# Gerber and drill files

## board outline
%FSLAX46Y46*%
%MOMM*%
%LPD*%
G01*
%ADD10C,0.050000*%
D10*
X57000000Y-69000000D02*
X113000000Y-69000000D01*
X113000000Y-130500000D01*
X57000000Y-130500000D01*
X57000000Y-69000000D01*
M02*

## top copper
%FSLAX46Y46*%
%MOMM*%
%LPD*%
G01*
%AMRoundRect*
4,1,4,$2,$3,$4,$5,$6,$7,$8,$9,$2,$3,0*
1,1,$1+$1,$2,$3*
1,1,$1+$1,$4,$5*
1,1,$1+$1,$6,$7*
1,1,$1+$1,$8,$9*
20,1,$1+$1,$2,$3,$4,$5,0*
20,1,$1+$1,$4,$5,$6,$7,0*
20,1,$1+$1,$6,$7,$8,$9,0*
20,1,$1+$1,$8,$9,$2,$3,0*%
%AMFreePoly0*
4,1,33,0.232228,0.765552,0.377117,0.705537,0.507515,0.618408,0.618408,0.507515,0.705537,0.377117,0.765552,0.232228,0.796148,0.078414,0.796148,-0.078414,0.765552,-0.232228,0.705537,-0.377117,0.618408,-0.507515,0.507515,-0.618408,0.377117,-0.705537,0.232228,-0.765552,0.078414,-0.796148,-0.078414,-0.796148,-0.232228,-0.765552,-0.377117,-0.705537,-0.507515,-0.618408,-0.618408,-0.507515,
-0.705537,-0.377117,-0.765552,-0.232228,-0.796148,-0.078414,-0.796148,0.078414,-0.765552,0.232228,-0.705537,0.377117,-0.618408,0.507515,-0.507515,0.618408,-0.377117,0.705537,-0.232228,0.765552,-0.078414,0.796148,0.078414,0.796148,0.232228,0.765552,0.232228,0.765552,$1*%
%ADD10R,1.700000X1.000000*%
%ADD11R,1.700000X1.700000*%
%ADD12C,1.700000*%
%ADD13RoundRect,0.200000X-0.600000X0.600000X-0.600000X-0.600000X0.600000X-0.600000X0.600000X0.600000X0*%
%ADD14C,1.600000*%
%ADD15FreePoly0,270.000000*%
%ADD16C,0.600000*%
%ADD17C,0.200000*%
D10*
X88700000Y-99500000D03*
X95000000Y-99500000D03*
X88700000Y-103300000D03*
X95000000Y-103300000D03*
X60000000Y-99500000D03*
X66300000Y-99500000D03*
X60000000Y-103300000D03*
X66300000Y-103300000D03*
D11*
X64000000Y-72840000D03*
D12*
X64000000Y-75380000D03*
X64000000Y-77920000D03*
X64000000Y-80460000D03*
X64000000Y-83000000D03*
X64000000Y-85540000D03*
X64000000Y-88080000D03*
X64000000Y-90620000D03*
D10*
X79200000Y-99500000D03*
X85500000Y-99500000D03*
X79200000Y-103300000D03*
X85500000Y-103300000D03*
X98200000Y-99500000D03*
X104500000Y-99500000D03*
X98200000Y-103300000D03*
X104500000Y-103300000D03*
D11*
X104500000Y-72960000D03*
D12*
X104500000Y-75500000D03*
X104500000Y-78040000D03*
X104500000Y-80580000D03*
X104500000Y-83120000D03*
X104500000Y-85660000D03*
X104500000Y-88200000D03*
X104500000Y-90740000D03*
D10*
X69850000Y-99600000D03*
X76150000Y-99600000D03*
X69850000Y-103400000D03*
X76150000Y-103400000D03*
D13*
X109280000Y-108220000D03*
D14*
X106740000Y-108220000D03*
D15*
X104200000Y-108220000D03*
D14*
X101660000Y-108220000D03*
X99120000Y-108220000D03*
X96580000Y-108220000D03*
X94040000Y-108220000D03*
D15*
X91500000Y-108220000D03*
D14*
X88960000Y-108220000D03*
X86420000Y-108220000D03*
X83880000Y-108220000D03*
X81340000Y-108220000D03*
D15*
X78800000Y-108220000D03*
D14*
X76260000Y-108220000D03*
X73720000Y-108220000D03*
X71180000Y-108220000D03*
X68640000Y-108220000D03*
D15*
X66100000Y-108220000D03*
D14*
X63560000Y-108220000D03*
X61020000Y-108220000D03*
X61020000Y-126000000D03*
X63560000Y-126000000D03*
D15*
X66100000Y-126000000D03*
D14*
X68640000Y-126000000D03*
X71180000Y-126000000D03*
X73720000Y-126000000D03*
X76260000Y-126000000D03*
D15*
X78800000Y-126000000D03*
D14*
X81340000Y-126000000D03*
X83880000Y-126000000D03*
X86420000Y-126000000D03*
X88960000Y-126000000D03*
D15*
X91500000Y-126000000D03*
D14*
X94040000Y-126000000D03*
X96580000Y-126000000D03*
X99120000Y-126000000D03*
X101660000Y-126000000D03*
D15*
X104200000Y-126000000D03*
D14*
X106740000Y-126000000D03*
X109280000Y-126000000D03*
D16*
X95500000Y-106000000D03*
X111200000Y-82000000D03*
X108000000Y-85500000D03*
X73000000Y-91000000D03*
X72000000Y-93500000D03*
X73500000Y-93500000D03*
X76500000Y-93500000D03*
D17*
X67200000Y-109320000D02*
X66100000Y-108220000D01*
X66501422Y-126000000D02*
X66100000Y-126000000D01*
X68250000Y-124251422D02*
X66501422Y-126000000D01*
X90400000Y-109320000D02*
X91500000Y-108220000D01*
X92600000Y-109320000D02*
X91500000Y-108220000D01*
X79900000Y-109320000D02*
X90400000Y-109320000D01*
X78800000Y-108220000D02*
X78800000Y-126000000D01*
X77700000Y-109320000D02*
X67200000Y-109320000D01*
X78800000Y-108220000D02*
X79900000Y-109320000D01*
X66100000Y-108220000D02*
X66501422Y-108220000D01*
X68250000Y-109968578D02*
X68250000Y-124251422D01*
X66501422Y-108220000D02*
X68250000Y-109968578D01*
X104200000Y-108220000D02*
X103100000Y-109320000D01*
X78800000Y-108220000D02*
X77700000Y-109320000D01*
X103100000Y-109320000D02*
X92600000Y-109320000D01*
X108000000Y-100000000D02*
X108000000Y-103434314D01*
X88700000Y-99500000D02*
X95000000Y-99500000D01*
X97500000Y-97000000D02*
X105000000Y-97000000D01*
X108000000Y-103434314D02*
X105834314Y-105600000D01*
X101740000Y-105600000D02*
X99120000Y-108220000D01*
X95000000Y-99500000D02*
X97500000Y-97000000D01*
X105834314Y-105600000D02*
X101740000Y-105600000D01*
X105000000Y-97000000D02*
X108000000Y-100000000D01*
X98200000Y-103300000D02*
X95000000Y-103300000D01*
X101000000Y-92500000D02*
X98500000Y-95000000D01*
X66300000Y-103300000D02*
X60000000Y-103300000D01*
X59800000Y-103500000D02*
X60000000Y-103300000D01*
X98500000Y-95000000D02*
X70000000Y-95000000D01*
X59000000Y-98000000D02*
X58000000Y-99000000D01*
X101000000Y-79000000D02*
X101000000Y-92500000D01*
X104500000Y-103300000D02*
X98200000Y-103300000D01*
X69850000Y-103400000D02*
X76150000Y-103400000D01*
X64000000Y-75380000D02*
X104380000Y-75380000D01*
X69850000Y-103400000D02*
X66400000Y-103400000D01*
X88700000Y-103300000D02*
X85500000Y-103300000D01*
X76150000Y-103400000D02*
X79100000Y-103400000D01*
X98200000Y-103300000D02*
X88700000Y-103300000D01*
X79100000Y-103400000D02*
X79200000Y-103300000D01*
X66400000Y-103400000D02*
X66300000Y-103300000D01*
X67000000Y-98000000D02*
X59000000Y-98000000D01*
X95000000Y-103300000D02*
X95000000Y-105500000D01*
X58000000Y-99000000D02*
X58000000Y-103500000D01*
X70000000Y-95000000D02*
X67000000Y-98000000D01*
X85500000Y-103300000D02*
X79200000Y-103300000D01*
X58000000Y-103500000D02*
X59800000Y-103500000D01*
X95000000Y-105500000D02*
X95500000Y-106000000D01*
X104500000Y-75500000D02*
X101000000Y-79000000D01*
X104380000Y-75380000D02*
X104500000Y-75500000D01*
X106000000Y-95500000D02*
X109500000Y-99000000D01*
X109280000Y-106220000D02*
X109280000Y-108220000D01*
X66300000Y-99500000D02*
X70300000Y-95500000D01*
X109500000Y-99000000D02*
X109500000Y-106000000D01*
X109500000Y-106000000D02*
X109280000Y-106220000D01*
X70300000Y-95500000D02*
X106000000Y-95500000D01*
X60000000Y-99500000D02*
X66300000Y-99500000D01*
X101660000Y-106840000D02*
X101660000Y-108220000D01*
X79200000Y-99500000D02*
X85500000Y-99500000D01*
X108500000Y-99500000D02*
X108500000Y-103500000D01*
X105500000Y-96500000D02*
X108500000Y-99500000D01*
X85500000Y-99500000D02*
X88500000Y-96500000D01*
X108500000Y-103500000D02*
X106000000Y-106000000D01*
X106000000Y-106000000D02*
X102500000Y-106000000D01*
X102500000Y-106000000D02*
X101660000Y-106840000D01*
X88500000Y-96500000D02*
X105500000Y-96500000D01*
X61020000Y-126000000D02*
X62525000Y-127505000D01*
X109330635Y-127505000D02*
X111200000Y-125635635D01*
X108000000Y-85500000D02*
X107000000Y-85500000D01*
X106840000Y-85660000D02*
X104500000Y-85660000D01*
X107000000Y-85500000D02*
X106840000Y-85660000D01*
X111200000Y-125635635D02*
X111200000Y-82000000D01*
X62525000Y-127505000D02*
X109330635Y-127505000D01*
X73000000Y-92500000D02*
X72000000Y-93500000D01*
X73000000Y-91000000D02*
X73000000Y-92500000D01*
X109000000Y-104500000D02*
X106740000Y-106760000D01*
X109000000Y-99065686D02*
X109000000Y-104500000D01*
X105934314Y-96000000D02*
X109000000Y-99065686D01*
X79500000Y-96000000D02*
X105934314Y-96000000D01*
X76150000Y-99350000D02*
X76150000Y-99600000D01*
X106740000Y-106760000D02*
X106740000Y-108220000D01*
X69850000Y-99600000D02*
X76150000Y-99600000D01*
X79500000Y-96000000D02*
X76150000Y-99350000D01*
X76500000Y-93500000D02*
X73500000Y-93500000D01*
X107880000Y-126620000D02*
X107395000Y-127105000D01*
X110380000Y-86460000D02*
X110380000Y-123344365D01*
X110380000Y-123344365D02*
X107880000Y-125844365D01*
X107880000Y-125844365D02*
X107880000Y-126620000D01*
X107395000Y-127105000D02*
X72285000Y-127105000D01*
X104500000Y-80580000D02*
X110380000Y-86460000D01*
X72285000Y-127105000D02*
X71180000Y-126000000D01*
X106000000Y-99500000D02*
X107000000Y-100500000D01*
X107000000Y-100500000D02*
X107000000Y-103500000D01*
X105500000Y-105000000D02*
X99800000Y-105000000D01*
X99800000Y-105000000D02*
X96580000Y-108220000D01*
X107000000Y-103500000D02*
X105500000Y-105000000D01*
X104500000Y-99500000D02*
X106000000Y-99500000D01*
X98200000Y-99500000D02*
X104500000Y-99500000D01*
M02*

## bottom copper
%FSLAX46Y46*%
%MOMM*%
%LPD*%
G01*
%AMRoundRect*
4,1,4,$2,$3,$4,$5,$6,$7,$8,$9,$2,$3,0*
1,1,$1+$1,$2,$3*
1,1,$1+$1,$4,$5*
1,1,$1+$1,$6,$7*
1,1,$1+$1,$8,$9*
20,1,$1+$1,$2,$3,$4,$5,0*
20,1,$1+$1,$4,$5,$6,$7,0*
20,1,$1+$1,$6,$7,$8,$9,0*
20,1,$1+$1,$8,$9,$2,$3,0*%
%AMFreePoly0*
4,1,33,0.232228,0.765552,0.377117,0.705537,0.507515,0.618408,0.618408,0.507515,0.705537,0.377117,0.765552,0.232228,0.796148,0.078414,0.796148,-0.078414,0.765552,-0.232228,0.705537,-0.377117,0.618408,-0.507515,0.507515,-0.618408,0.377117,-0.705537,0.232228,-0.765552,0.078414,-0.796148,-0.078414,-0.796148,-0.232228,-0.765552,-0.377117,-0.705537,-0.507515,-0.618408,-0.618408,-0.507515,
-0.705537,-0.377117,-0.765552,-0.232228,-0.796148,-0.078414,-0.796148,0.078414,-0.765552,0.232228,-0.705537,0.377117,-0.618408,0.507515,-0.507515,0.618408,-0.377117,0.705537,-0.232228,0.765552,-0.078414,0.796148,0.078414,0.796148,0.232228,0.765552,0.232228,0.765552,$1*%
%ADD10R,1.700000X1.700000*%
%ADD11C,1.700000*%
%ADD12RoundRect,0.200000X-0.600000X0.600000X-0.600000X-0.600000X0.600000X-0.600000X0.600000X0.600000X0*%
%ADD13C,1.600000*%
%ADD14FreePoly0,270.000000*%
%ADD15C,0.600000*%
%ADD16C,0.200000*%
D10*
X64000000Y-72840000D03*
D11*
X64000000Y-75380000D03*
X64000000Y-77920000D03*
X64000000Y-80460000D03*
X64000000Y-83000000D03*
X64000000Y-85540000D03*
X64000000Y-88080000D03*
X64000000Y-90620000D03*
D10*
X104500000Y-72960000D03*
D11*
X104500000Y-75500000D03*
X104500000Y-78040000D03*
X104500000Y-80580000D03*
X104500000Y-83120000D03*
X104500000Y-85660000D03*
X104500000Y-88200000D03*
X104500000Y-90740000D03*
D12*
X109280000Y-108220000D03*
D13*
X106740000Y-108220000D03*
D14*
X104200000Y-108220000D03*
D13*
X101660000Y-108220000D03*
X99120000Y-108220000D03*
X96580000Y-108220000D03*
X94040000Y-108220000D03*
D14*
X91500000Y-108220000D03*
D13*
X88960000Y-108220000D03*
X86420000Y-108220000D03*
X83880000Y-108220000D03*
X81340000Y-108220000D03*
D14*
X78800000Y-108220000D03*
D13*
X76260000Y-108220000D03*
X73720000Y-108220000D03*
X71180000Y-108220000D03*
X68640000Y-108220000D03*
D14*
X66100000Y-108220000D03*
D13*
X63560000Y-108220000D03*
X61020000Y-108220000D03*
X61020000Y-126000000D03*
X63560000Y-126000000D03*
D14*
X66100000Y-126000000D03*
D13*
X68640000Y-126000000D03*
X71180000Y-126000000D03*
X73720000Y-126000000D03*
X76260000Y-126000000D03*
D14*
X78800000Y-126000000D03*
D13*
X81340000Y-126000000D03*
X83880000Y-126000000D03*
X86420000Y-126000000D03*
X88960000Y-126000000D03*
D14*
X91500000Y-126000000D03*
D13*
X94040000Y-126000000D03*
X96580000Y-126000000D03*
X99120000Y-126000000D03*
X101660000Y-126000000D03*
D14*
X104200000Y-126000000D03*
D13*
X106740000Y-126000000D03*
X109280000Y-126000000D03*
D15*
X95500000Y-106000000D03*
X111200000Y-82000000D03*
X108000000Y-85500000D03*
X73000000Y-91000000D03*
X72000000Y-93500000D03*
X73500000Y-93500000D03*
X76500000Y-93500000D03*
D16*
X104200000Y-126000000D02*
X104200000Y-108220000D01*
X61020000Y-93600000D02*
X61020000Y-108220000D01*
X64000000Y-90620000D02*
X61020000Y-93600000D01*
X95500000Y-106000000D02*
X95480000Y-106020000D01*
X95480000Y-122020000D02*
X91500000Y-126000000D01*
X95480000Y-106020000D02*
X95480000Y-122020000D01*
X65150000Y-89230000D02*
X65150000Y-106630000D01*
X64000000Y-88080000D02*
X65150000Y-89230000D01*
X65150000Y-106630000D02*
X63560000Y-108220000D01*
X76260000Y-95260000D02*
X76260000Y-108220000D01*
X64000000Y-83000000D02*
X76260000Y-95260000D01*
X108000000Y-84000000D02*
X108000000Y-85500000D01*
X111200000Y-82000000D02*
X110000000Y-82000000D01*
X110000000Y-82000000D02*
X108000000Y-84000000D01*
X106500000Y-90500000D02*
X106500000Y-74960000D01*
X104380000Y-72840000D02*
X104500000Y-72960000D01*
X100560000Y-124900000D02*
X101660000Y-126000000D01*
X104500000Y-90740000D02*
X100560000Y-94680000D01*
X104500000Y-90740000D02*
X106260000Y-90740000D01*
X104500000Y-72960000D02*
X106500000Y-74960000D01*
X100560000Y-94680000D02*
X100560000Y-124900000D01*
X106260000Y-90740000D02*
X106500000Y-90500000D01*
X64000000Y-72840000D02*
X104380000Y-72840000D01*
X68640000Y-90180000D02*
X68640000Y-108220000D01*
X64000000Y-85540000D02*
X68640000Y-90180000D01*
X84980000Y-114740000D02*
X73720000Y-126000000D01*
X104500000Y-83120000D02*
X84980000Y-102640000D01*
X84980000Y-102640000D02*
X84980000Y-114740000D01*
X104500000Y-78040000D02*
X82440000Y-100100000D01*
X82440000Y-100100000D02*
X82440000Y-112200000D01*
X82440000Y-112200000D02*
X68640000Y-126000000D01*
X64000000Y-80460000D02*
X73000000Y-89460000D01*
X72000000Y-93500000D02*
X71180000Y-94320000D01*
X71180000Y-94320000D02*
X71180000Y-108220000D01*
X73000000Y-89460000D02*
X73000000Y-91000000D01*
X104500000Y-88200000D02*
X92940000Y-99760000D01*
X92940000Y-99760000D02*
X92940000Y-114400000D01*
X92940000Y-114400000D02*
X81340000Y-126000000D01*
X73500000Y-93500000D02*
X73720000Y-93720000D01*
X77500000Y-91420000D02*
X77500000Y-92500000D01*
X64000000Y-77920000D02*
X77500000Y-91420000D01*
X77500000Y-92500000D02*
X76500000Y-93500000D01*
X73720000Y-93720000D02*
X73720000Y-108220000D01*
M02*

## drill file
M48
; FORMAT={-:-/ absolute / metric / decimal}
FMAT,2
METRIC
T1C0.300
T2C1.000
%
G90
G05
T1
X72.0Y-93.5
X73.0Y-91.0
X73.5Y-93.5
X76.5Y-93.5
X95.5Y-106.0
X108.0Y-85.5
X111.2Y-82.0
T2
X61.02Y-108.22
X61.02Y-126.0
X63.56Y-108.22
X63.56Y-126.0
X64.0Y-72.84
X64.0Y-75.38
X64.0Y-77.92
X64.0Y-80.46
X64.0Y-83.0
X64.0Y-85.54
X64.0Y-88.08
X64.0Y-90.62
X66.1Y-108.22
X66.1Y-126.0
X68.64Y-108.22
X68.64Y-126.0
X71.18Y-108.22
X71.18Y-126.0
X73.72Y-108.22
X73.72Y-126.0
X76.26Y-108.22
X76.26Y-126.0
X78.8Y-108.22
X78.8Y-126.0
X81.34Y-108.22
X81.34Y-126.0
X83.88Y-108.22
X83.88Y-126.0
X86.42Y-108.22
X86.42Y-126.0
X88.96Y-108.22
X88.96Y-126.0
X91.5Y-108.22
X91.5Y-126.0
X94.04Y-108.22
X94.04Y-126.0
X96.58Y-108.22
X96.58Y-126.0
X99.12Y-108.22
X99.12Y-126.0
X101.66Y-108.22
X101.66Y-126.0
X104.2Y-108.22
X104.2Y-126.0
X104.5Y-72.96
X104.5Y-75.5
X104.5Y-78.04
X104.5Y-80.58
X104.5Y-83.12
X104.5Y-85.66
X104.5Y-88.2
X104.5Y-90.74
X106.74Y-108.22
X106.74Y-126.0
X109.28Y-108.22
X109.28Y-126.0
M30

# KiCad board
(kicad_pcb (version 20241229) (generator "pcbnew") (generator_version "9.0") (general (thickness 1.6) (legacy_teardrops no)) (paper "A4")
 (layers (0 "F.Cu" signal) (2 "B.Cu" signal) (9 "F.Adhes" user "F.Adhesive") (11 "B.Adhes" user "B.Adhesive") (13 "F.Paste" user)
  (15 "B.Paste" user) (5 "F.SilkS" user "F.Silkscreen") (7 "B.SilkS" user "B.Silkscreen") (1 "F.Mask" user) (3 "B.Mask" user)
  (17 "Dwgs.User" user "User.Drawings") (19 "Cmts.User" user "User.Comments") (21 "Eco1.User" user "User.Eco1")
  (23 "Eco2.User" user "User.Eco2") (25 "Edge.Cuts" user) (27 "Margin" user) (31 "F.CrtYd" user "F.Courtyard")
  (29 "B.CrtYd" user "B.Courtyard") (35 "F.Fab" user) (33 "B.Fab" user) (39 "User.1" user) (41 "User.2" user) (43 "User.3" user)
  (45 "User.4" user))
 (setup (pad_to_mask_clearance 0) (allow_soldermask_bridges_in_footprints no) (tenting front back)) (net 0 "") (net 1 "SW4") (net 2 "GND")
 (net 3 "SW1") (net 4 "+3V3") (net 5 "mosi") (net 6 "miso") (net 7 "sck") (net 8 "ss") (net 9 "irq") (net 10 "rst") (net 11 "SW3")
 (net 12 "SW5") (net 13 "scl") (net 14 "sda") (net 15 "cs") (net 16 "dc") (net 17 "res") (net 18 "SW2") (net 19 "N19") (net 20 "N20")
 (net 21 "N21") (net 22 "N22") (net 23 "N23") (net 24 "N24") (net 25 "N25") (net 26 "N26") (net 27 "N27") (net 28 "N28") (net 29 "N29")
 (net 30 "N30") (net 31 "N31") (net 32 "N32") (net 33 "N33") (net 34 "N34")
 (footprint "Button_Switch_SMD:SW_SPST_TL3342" (layer "F.Cu") (at 91.85 101.4)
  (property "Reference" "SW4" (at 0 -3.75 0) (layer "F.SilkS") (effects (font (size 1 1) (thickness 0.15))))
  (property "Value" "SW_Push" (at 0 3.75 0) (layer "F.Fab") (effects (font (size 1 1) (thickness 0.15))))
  (pad "1" smd rect (at -3.15 -1.9) (size 1.7 1) (layers "F.Cu" "F.Mask" "F.Paste") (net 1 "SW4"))
  (pad "1" smd rect (at 3.15 -1.9) (size 1.7 1) (layers "F.Cu" "F.Mask" "F.Paste") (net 1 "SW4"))
  (pad "2" smd rect (at -3.15 1.9) (size 1.7 1) (layers "F.Cu" "F.Mask" "F.Paste") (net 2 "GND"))
  (pad "2" smd rect (at 3.15 1.9) (size 1.7 1) (layers "F.Cu" "F.Mask" "F.Paste") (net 2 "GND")))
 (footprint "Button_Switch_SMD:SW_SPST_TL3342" (layer "F.Cu") (at 63.15 101.4)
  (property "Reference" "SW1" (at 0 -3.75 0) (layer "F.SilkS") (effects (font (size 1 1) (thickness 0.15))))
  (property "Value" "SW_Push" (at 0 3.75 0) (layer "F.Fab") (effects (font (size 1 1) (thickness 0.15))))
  (pad "1" smd rect (at -3.15 -1.9) (size 1.7 1) (layers "F.Cu" "F.Mask" "F.Paste") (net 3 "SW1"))
  (pad "1" smd rect (at 3.15 -1.9) (size 1.7 1) (layers "F.Cu" "F.Mask" "F.Paste") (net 3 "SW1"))
  (pad "2" smd rect (at -3.15 1.9) (size 1.7 1) (layers "F.Cu" "F.Mask" "F.Paste") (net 2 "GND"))
  (pad "2" smd rect (at 3.15 1.9) (size 1.7 1) (layers "F.Cu" "F.Mask" "F.Paste") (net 2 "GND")))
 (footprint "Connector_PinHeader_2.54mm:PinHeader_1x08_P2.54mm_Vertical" (layer "F.Cu") (at 64 72.84)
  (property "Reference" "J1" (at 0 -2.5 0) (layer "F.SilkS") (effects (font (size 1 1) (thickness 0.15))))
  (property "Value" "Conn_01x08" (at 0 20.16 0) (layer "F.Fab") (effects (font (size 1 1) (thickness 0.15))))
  (pad "1" thru_hole rect (at 0 0) (size 1.7 1.7) (drill 1) (layers "*.Cu" "*.Mask") (remove_unused_layers no) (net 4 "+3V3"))
  (pad "2" thru_hole circle (at 0 2.54) (size 1.7 1.7) (drill 1) (layers "*.Cu" "*.Mask") (remove_unused_layers no) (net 2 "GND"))
  (pad "3" thru_hole circle (at 0 5.08) (size 1.7 1.7) (drill 1) (layers "*.Cu" "*.Mask") (remove_unused_layers no) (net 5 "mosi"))
  (pad "4" thru_hole circle (at 0 7.62) (size 1.7 1.7) (drill 1) (layers "*.Cu" "*.Mask") (remove_unused_layers no) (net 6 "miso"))
  (pad "5" thru_hole circle (at 0 10.16) (size 1.7 1.7) (drill 1) (layers "*.Cu" "*.Mask") (remove_unused_layers no) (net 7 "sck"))
  (pad "6" thru_hole circle (at 0 12.7) (size 1.7 1.7) (drill 1) (layers "*.Cu" "*.Mask") (remove_unused_layers no) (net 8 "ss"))
  (pad "7" thru_hole circle (at 0 15.24) (size 1.7 1.7) (drill 1) (layers "*.Cu" "*.Mask") (remove_unused_layers no) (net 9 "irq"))
  (pad "8" thru_hole circle (at 0 17.78) (size 1.7 1.7) (drill 1) (layers "*.Cu" "*.Mask") (remove_unused_layers no) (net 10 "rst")))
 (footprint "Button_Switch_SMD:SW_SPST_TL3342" (layer "F.Cu") (at 82.35 101.4)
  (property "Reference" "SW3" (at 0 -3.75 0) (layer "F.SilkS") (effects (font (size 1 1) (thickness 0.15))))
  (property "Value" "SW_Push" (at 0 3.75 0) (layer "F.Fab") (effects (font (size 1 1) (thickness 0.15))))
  (pad "1" smd rect (at -3.15 -1.9) (size 1.7 1) (layers "F.Cu" "F.Mask" "F.Paste") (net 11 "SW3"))
  (pad "1" smd rect (at 3.15 -1.9) (size 1.7 1) (layers "F.Cu" "F.Mask" "F.Paste") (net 11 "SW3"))
  (pad "2" smd rect (at -3.15 1.9) (size 1.7 1) (layers "F.Cu" "F.Mask" "F.Paste") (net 2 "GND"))
  (pad "2" smd rect (at 3.15 1.9) (size 1.7 1) (layers "F.Cu" "F.Mask" "F.Paste") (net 2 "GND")))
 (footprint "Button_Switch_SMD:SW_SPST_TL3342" (layer "F.Cu") (at 101.35 101.4)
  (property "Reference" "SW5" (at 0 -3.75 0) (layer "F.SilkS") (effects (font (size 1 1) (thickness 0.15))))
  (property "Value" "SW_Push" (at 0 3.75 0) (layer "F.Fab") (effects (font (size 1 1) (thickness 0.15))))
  (pad "1" smd rect (at -3.15 -1.9) (size 1.7 1) (layers "F.Cu" "F.Mask" "F.Paste") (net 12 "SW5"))
  (pad "1" smd rect (at 3.15 -1.9) (size 1.7 1) (layers "F.Cu" "F.Mask" "F.Paste") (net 12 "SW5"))
  (pad "2" smd rect (at -3.15 1.9) (size 1.7 1) (layers "F.Cu" "F.Mask" "F.Paste") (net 2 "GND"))
  (pad "2" smd rect (at 3.15 1.9) (size 1.7 1) (layers "F.Cu" "F.Mask" "F.Paste") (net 2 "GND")))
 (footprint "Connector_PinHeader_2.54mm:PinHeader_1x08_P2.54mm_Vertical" (layer "F.Cu") (at 104.5 72.96)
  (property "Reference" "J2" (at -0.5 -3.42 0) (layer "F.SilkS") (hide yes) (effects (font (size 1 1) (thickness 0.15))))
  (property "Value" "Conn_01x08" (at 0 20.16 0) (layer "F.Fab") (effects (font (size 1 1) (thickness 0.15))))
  (pad "1" thru_hole rect (at 0 0) (size 1.7 1.7) (drill 1) (layers "*.Cu" "*.Mask") (remove_unused_layers no) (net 4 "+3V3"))
  (pad "2" thru_hole circle (at 0 2.54) (size 1.7 1.7) (drill 1) (layers "*.Cu" "*.Mask") (remove_unused_layers no) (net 2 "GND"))
  (pad "3" thru_hole circle (at 0 5.08) (size 1.7 1.7) (drill 1) (layers "*.Cu" "*.Mask") (remove_unused_layers no) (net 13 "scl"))
  (pad "4" thru_hole circle (at 0 7.62) (size 1.7 1.7) (drill 1) (layers "*.Cu" "*.Mask") (remove_unused_layers no) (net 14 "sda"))
  (pad "5" thru_hole circle (at 0 10.16) (size 1.7 1.7) (drill 1) (layers "*.Cu" "*.Mask") (remove_unused_layers no) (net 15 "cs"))
  (pad "6" thru_hole circle (at 0 12.7) (size 1.7 1.7) (drill 1) (layers "*.Cu" "*.Mask") (remove_unused_layers no) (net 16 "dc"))
  (pad "7" thru_hole circle (at 0 15.24) (size 1.7 1.7) (drill 1) (layers "*.Cu" "*.Mask") (remove_unused_layers no) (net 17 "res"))
  (pad "8" thru_hole circle (at 0 17.78) (size 1.7 1.7) (drill 1) (layers "*.Cu" "*.Mask") (remove_unused_layers no) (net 4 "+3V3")))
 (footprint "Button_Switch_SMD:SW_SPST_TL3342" (layer "F.Cu") (at 73 101.5)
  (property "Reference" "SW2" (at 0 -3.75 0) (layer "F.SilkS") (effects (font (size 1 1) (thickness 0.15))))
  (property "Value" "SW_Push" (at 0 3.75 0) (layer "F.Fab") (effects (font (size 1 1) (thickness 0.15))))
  (pad "1" smd rect (at -3.15 -1.9) (size 1.7 1) (layers "F.Cu" "F.Mask" "F.Paste") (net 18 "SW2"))
  (pad "1" smd rect (at 3.15 -1.9) (size 1.7 1) (layers "F.Cu" "F.Mask" "F.Paste") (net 18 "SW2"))
  (pad "2" smd rect (at -3.15 1.9) (size 1.7 1) (layers "F.Cu" "F.Mask" "F.Paste") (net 2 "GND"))
  (pad "2" smd rect (at 3.15 1.9) (size 1.7 1) (layers "F.Cu" "F.Mask" "F.Paste") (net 2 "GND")))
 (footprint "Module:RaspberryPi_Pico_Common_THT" (layer "F.Cu") (at 109.28 108.22 -90)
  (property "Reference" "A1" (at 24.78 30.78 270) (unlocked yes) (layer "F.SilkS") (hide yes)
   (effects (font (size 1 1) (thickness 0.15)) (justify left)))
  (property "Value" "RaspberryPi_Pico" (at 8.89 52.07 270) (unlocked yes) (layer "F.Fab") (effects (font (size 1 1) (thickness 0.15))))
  (pad "1" thru_hole roundrect (at 0 0 270) (size 1.6 1.6) (drill 1) (layers "*.Cu" "*.Mask") (remove_unused_layers no)
   (roundrect_rratio 0.125) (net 3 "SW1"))
  (pad "2" thru_hole circle (at 0 2.54 270) (size 1.6 1.6) (drill 1) (layers "*.Cu" "*.Mask") (remove_unused_layers no) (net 18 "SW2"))
  (pad "3" thru_hole custom (at 0 5.08 270) (size 1.6 1.6) (drill 1) (layers "*.Cu" "*.Mask") (remove_unused_layers no) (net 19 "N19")
   (options (clearance outline) (anchor circle)) (primitives))
  (pad "4" thru_hole circle (at 0 7.62 270) (size 1.6 1.6) (drill 1) (layers "*.Cu" "*.Mask") (remove_unused_layers no) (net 11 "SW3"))
  (pad "5" thru_hole circle (at 0 10.16 270) (size 1.6 1.6) (drill 1) (layers "*.Cu" "*.Mask") (remove_unused_layers no) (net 1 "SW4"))
  (pad "6" thru_hole circle (at 0 12.7 270) (size 1.6 1.6) (drill 1) (layers "*.Cu" "*.Mask") (remove_unused_layers no) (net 12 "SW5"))
  (pad "7" thru_hole circle (at 0 15.24 270) (size 1.6 1.6) (drill 1) (layers "*.Cu" "*.Mask") (remove_unused_layers no) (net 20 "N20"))
  (pad "8" thru_hole custom (at 0 17.78 270) (size 1.6 1.6) (drill 1) (layers "*.Cu" "*.Mask") (remove_unused_layers no) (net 19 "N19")
   (options (clearance outline) (anchor circle)) (primitives))
  (pad "9" thru_hole circle (at 0 20.32 270) (size 1.6 1.6) (drill 1) (layers "*.Cu" "*.Mask") (remove_unused_layers no) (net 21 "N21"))
  (pad "10" thru_hole circle (at 0 22.86 270) (size 1.6 1.6) (drill 1) (layers "*.Cu" "*.Mask") (remove_unused_layers no) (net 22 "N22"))
  (pad "11" thru_hole circle (at 0 25.4 270) (size 1.6 1.6) (drill 1) (layers "*.Cu" "*.Mask") (remove_unused_layers no) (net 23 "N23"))
  (pad "12" thru_hole circle (at 0 27.94 270) (size 1.6 1.6) (drill 1) (layers "*.Cu" "*.Mask") (remove_unused_layers no) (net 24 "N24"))
  (pad "13" thru_hole custom (at 0 30.48 270) (size 1.6 1.6) (drill 1) (layers "*.Cu" "*.Mask") (remove_unused_layers no) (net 19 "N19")
   (options (clearance outline) (anchor circle)) (primitives))
  (pad "14" thru_hole circle (at 0 33.02 270) (size 1.6 1.6) (drill 1) (layers "*.Cu" "*.Mask") (remove_unused_layers no) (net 7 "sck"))
  (pad "15" thru_hole circle (at 0 35.56 270) (size 1.6 1.6) (drill 1) (layers "*.Cu" "*.Mask") (remove_unused_layers no) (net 5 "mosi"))
  (pad "16" thru_hole circle (at 0 38.1 270) (size 1.6 1.6) (drill 1) (layers "*.Cu" "*.Mask") (remove_unused_layers no) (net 6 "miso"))
  (pad "17" thru_hole circle (at 0 40.64 270) (size 1.6 1.6) (drill 1) (layers "*.Cu" "*.Mask") (remove_unused_layers no) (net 8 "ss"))
  (pad "18" thru_hole custom (at 0 43.18 270) (size 1.6 1.6) (drill 1) (layers "*.Cu" "*.Mask") (remove_unused_layers no) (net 19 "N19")
   (options (clearance outline) (anchor circle)) (primitives))
  (pad "19" thru_hole circle (at 0 45.72 270) (size 1.6 1.6) (drill 1) (layers "*.Cu" "*.Mask") (remove_unused_layers no) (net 9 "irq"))
  (pad "20" thru_hole circle (at 0 48.26 270) (size 1.6 1.6) (drill 1) (layers "*.Cu" "*.Mask") (remove_unused_layers no) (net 10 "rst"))
  (pad "21" thru_hole circle (at 17.78 48.26 270) (size 1.6 1.6) (drill 1) (layers "*.Cu" "*.Mask") (remove_unused_layers no) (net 16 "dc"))
  (pad "22" thru_hole circle (at 17.78 45.72 270) (size 1.6 1.6) (drill 1) (layers "*.Cu" "*.Mask") (remove_unused_layers no) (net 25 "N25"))
  (pad "23" thru_hole custom (at 17.78 43.18 270) (size 1.6 1.6) (drill 1) (layers "*.Cu" "*.Mask") (remove_unused_layers no) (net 19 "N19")
   (options (clearance outline) (anchor circle)) (primitives))
  (pad "24" thru_hole circle (at 17.78 40.64 270) (size 1.6 1.6) (drill 1) (layers "*.Cu" "*.Mask") (remove_unused_layers no) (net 13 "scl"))
  (pad "25" thru_hole circle (at 17.78 38.1 270) (size 1.6 1.6) (drill 1) (layers "*.Cu" "*.Mask") (remove_unused_layers no) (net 14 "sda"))
  (pad "26" thru_hole circle (at 17.78 35.56 270) (size 1.6 1.6) (drill 1) (layers "*.Cu" "*.Mask") (remove_unused_layers no) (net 15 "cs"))
  (pad "27" thru_hole circle (at 17.78 33.02 270) (size 1.6 1.6) (drill 1) (layers "*.Cu" "*.Mask") (remove_unused_layers no) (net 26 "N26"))
  (pad "28" thru_hole custom (at 17.78 30.48 270) (size 1.6 1.6) (drill 1) (layers "*.Cu" "*.Mask") (remove_unused_layers no) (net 19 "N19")
   (options (clearance outline) (anchor circle)) (primitives))
  (pad "29" thru_hole circle (at 17.78 27.94 270) (size 1.6 1.6) (drill 1) (layers "*.Cu" "*.Mask") (remove_unused_layers no) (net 17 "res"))
  (pad "30" thru_hole circle (at 17.78 25.4 270) (size 1.6 1.6) (drill 1) (layers "*.Cu" "*.Mask") (remove_unused_layers no) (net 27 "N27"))
  (pad "31" thru_hole circle (at 17.78 22.86 270) (size 1.6 1.6) (drill 1) (layers "*.Cu" "*.Mask") (remove_unused_layers no) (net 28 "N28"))
  (pad "32" thru_hole circle (at 17.78 20.32 270) (size 1.6 1.6) (drill 1) (layers "*.Cu" "*.Mask") (remove_unused_layers no) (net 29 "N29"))
  (pad "33" thru_hole custom (at 17.78 17.78 270) (size 1.6 1.6) (drill 1) (layers "*.Cu" "*.Mask") (remove_unused_layers no) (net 2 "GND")
   (options (clearance outline) (anchor circle)) (primitives))
  (pad "34" thru_hole circle (at 17.78 15.24 270) (size 1.6 1.6) (drill 1) (layers "*.Cu" "*.Mask") (remove_unused_layers no) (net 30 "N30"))
  (pad "35" thru_hole circle (at 17.78 12.7 270) (size 1.6 1.6) (drill 1) (layers "*.Cu" "*.Mask") (remove_unused_layers no) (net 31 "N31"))
  (pad "36" thru_hole circle (at 17.78 10.16 270) (size 1.6 1.6) (drill 1) (layers "*.Cu" "*.Mask") (remove_unused_layers no) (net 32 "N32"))
  (pad "37" thru_hole circle (at 17.78 7.62 270) (size 1.6 1.6) (drill 1) (layers "*.Cu" "*.Mask") (remove_unused_layers no) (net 4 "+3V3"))
  (pad "38" thru_hole custom (at 17.78 5.08 270) (size 1.6 1.6) (drill 1) (layers "*.Cu" "*.Mask") (remove_unused_layers no) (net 19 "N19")
   (options (clearance outline) (anchor circle)) (primitives))
  (pad "39" thru_hole circle (at 17.78 2.54 270) (size 1.6 1.6) (drill 1) (layers "*.Cu" "*.Mask") (remove_unused_layers no) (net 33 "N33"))
  (pad "40" thru_hole circle (at 17.78 0 270) (size 1.6 1.6) (drill 1) (layers "*.Cu" "*.Mask") (remove_unused_layers no) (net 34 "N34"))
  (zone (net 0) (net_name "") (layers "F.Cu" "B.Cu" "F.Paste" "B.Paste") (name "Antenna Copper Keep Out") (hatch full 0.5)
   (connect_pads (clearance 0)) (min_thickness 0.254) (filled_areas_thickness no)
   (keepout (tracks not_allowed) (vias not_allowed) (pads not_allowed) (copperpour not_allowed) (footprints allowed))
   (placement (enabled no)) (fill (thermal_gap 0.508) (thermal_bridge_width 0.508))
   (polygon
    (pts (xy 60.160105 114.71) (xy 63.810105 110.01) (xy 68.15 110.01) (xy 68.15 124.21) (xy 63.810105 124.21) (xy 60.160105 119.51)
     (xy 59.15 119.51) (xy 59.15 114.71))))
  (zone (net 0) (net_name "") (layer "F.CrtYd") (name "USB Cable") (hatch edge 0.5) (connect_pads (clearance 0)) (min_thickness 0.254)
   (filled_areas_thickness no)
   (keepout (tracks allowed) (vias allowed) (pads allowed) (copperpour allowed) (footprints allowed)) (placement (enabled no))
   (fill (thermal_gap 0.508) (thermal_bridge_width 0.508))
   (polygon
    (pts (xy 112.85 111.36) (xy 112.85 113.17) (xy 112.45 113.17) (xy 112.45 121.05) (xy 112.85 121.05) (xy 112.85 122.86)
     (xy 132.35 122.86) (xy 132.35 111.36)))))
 (gr_rect (start 57 69) (end 113 130.5) (stroke (width 0.05) (type default)) (fill no) (layer "Edge.Cuts"))
 (segment (start 67.2 109.32) (end 66.1 108.22) (width 0.2) (layer "F.Cu") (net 19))
 (segment (start 66.501422 126) (end 66.1 126) (width 0.2) (layer "F.Cu") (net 19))
 (segment (start 68.25 124.251422) (end 66.501422 126) (width 0.2) (layer "F.Cu") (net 19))
 (segment (start 90.4 109.32) (end 91.5 108.22) (width 0.2) (layer "F.Cu") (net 19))
 (segment (start 92.6 109.32) (end 91.5 108.22) (width 0.2) (layer "F.Cu") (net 19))
 (segment (start 79.9 109.32) (end 90.4 109.32) (width 0.2) (layer "F.Cu") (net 19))
 (segment (start 78.8 108.22) (end 78.8 126) (width 0.2) (layer "F.Cu") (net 19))
 (segment (start 77.7 109.32) (end 67.2 109.32) (width 0.2) (layer "F.Cu") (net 19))
 (segment (start 78.8 108.22) (end 79.9 109.32) (width 0.2) (layer "F.Cu") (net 19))
 (segment (start 66.1 108.22) (end 66.501422 108.22) (width 0.2) (layer "F.Cu") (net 19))
 (segment (start 68.25 109.968578) (end 68.25 124.251422) (width 0.2) (layer "F.Cu") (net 19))
 (segment (start 66.501422 108.22) (end 68.25 109.968578) (width 0.2) (layer "F.Cu") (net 19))
 (segment (start 104.2 108.22) (end 103.1 109.32) (width 0.2) (layer "F.Cu") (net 19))
 (segment (start 78.8 108.22) (end 77.7 109.32) (width 0.2) (layer "F.Cu") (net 19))
 (segment (start 103.1 109.32) (end 92.6 109.32) (width 0.2) (layer "F.Cu") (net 19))
 (segment (start 104.2 126) (end 104.2 108.22) (width 0.2) (layer "B.Cu") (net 19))
 (segment (start 61.02 93.6) (end 61.02 108.22) (width 0.2) (layer "B.Cu") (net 10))
 (segment (start 64 90.62) (end 61.02 93.6) (width 0.2) (layer "B.Cu") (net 10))
 (segment (start 108 100) (end 108 103.434314) (width 0.2) (layer "F.Cu") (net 1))
 (segment (start 88.7 99.5) (end 95 99.5) (width 0.2) (layer "F.Cu") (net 1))
 (segment (start 97.5 97) (end 105 97) (width 0.2) (layer "F.Cu") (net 1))
 (segment (start 108 103.434314) (end 105.834314 105.6) (width 0.2) (layer "F.Cu") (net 1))
 (segment (start 101.74 105.6) (end 99.12 108.22) (width 0.2) (layer "F.Cu") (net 1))
 (segment (start 95 99.5) (end 97.5 97) (width 0.2) (layer "F.Cu") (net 1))
 (segment (start 105.834314 105.6) (end 101.74 105.6) (width 0.2) (layer "F.Cu") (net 1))
 (segment (start 105 97) (end 108 100) (width 0.2) (layer "F.Cu") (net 1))
 (segment (start 98.2 103.3) (end 95 103.3) (width 0.2) (layer "F.Cu") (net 2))
 (segment (start 101 92.5) (end 98.5 95) (width 0.2) (layer "F.Cu") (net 2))
 (segment (start 66.3 103.3) (end 60 103.3) (width 0.2) (layer "F.Cu") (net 2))
 (segment (start 59.8 103.5) (end 60 103.3) (width 0.2) (layer "F.Cu") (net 2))
 (segment (start 98.5 95) (end 70 95) (width 0.2) (layer "F.Cu") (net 2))
 (segment (start 59 98) (end 58 99) (width 0.2) (layer "F.Cu") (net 2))
 (segment (start 101 79) (end 101 92.5) (width 0.2) (layer "F.Cu") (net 2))
 (segment (start 104.5 103.3) (end 98.2 103.3) (width 0.2) (layer "F.Cu") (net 2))
 (segment (start 69.85 103.4) (end 76.15 103.4) (width 0.2) (layer "F.Cu") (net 2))
 (segment (start 64 75.38) (end 104.38 75.38) (width 0.2) (layer "F.Cu") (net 2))
 (segment (start 69.85 103.4) (end 66.4 103.4) (width 0.2) (layer "F.Cu") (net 2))
 (segment (start 88.7 103.3) (end 85.5 103.3) (width 0.2) (layer "F.Cu") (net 2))
 (segment (start 76.15 103.4) (end 79.1 103.4) (width 0.2) (layer "F.Cu") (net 2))
 (segment (start 98.2 103.3) (end 88.7 103.3) (width 0.2) (layer "F.Cu") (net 2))
 (segment (start 79.1 103.4) (end 79.2 103.3) (width 0.2) (layer "F.Cu") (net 2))
 (segment (start 66.4 103.4) (end 66.3 103.3) (width 0.2) (layer "F.Cu") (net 2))
 (segment (start 67 98) (end 59 98) (width 0.2) (layer "F.Cu") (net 2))
 (segment (start 95 103.3) (end 95 105.5) (width 0.2) (layer "F.Cu") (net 2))
 (segment (start 58 99) (end 58 103.5) (width 0.2) (layer "F.Cu") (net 2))
 (segment (start 70 95) (end 67 98) (width 0.2) (layer "F.Cu") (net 2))
 (segment (start 85.5 103.3) (end 79.2 103.3) (width 0.2) (layer "F.Cu") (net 2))
 (segment (start 58 103.5) (end 59.8 103.5) (width 0.2) (layer "F.Cu") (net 2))
 (segment (start 95 105.5) (end 95.5 106) (width 0.2) (layer "F.Cu") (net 2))
 (segment (start 104.5 75.5) (end 101 79) (width 0.2) (layer "F.Cu") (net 2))
 (segment (start 104.38 75.38) (end 104.5 75.5) (width 0.2) (layer "F.Cu") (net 2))
 (via (at 95.5 106) (size 0.6) (drill 0.3) (layers "F.Cu" "B.Cu") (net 2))
 (segment (start 95.5 106) (end 95.48 106.02) (width 0.2) (layer "B.Cu") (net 2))
 (segment (start 95.48 122.02) (end 91.5 126) (width 0.2) (layer "B.Cu") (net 2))
 (segment (start 95.48 106.02) (end 95.48 122.02) (width 0.2) (layer "B.Cu") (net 2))
 (segment (start 106 95.5) (end 109.5 99) (width 0.2) (layer "F.Cu") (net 3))
 (segment (start 109.28 106.22) (end 109.28 108.22) (width 0.2) (layer "F.Cu") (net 3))
 (segment (start 66.3 99.5) (end 70.3 95.5) (width 0.2) (layer "F.Cu") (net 3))
 (segment (start 109.5 99) (end 109.5 106) (width 0.2) (layer "F.Cu") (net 3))
 (segment (start 109.5 106) (end 109.28 106.22) (width 0.2) (layer "F.Cu") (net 3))
 (segment (start 70.3 95.5) (end 106 95.5) (width 0.2) (layer "F.Cu") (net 3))
 (segment (start 60 99.5) (end 66.3 99.5) (width 0.2) (layer "F.Cu") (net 3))
 (segment (start 65.15 89.23) (end 65.15 106.63) (width 0.2) (layer "B.Cu") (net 9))
 (segment (start 64 88.08) (end 65.15 89.23) (width 0.2) (layer "B.Cu") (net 9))
 (segment (start 65.15 106.63) (end 63.56 108.22) (width 0.2) (layer "B.Cu") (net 9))
 (segment (start 101.66 106.84) (end 101.66 108.22) (width 0.2) (layer "F.Cu") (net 11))
 (segment (start 79.2 99.5) (end 85.5 99.5) (width 0.2) (layer "F.Cu") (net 11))
 (segment (start 108.5 99.5) (end 108.5 103.5) (width 0.2) (layer "F.Cu") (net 11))
 (segment (start 105.5 96.5) (end 108.5 99.5) (width 0.2) (layer "F.Cu") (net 11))
 (segment (start 85.5 99.5) (end 88.5 96.5) (width 0.2) (layer "F.Cu") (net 11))
 (segment (start 108.5 103.5) (end 106 106) (width 0.2) (layer "F.Cu") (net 11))
 (segment (start 106 106) (end 102.5 106) (width 0.2) (layer "F.Cu") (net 11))
 (segment (start 102.5 106) (end 101.66 106.84) (width 0.2) (layer "F.Cu") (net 11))
 (segment (start 88.5 96.5) (end 105.5 96.5) (width 0.2) (layer "F.Cu") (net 11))
 (segment (start 76.26 95.26) (end 76.26 108.22) (width 0.2) (layer "B.Cu") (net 7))
 (segment (start 64 83) (end 76.26 95.26) (width 0.2) (layer "B.Cu") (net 7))
 (segment (start 61.02 126) (end 62.525 127.505) (width 0.2) (layer "F.Cu") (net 16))
 (segment (start 109.330635 127.505) (end 111.2 125.635635) (width 0.2) (layer "F.Cu") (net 16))
 (segment (start 108 85.5) (end 107 85.5) (width 0.2) (layer "F.Cu") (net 16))
 (segment (start 106.84 85.66) (end 104.5 85.66) (width 0.2) (layer "F.Cu") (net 16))
 (segment (start 107 85.5) (end 106.84 85.66) (width 0.2) (layer "F.Cu") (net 16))
 (segment (start 111.2 125.635635) (end 111.2 82) (width 0.2) (layer "F.Cu") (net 16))
 (segment (start 62.525 127.505) (end 109.330635 127.505) (width 0.2) (layer "F.Cu") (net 16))
 (via (at 111.2 82) (size 0.6) (drill 0.3) (layers "F.Cu" "B.Cu") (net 16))
 (via (at 108 85.5) (size 0.6) (drill 0.3) (layers "F.Cu" "B.Cu") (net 16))
 (segment (start 108 84) (end 108 85.5) (width 0.2) (layer "B.Cu") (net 16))
 (segment (start 111.2 82) (end 110 82) (width 0.2) (layer "B.Cu") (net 16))
 (segment (start 110 82) (end 108 84) (width 0.2) (layer "B.Cu") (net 16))
 (segment (start 106.5 90.5) (end 106.5 74.96) (width 0.2) (layer "B.Cu") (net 4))
 (segment (start 104.38 72.84) (end 104.5 72.96) (width 0.2) (layer "B.Cu") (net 4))
 (segment (start 100.56 124.9) (end 101.66 126) (width 0.2) (layer "B.Cu") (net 4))
 (segment (start 104.5 90.74) (end 100.56 94.68) (width 0.2) (layer "B.Cu") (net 4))
 (segment (start 104.5 90.74) (end 106.26 90.74) (width 0.2) (layer "B.Cu") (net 4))
 (segment (start 104.5 72.96) (end 106.5 74.96) (width 0.2) (layer "B.Cu") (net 4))
 (segment (start 100.56 94.68) (end 100.56 124.9) (width 0.2) (layer "B.Cu") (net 4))
 (segment (start 106.26 90.74) (end 106.5 90.5) (width 0.2) (layer "B.Cu") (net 4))
 (segment (start 64 72.84) (end 104.38 72.84) (width 0.2) (layer "B.Cu") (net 4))
 (segment (start 68.64 90.18) (end 68.64 108.22) (width 0.2) (layer "B.Cu") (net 8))
 (segment (start 64 85.54) (end 68.64 90.18) (width 0.2) (layer "B.Cu") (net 8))
 (segment (start 84.98 114.74) (end 73.72 126) (width 0.2) (layer "B.Cu") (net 15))
 (segment (start 104.5 83.12) (end 84.98 102.64) (width 0.2) (layer "B.Cu") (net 15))
 (segment (start 84.98 102.64) (end 84.98 114.74) (width 0.2) (layer "B.Cu") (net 15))
 (segment (start 104.5 78.04) (end 82.44 100.1) (width 0.2) (layer "B.Cu") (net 13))
 (segment (start 82.44 100.1) (end 82.44 112.2) (width 0.2) (layer "B.Cu") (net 13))
 (segment (start 82.44 112.2) (end 68.64 126) (width 0.2) (layer "B.Cu") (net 13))
 (segment (start 73 92.5) (end 72 93.5) (width 0.2) (layer "F.Cu") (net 6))
 (segment (start 73 91) (end 73 92.5) (width 0.2) (layer "F.Cu") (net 6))
 (via (at 73 91) (size 0.6) (drill 0.3) (layers "F.Cu" "B.Cu") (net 6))
 (via (at 72 93.5) (size 0.6) (drill 0.3) (layers "F.Cu" "B.Cu") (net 6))
 (segment (start 64 80.46) (end 73 89.46) (width 0.2) (layer "B.Cu") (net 6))
 (segment (start 72 93.5) (end 71.18 94.32) (width 0.2) (layer "B.Cu") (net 6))
 (segment (start 71.18 94.32) (end 71.18 108.22) (width 0.2) (layer "B.Cu") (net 6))
 (segment (start 73 89.46) (end 73 91) (width 0.2) (layer "B.Cu") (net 6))
 (segment (start 109 104.5) (end 106.74 106.76) (width 0.2) (layer "F.Cu") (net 18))
 (segment (start 109 99.065686) (end 109 104.5) (width 0.2) (layer "F.Cu") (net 18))
 (segment (start 105.934314 96) (end 109 99.065686) (width 0.2) (layer "F.Cu") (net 18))
 (segment (start 79.5 96) (end 105.934314 96) (width 0.2) (layer "F.Cu") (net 18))
 (segment (start 76.15 99.35) (end 76.15 99.6) (width 0.2) (layer "F.Cu") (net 18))
 (segment (start 106.74 106.76) (end 106.74 108.22) (width 0.2) (layer "F.Cu") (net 18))
 (segment (start 69.85 99.6) (end 76.15 99.6) (width 0.2) (layer "F.Cu") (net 18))
 (segment (start 79.5 96) (end 76.15 99.35) (width 0.2) (layer "F.Cu") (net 18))
 (segment (start 104.5 88.2) (end 92.94 99.76) (width 0.2) (layer "B.Cu") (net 17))
 (segment (start 92.94 99.76) (end 92.94 114.4) (width 0.2) (layer "B.Cu") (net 17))
 (segment (start 92.94 114.4) (end 81.34 126) (width 0.2) (layer "B.Cu") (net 17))
 (segment (start 76.5 93.5) (end 73.5 93.5) (width 0.2) (layer "F.Cu") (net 5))
 (via (at 73.5 93.5) (size 0.6) (drill 0.3) (layers "F.Cu" "B.Cu") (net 5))
 (via (at 76.5 93.5) (size 0.6) (drill 0.3) (layers "F.Cu" "B.Cu") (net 5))
 (segment (start 73.5 93.5) (end 73.72 93.72) (width 0.2) (layer "B.Cu") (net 5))
 (segment (start 77.5 91.42) (end 77.5 92.5) (width 0.2) (layer "B.Cu") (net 5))
 (segment (start 64 77.92) (end 77.5 91.42) (width 0.2) (layer "B.Cu") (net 5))
 (segment (start 77.5 92.5) (end 76.5 93.5) (width 0.2) (layer "B.Cu") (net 5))
 (segment (start 73.72 93.72) (end 73.72 108.22) (width 0.2) (layer "B.Cu") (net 5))
 (segment (start 107.88 126.62) (end 107.395 127.105) (width 0.2) (layer "F.Cu") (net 14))
 (segment (start 110.38 86.46) (end 110.38 123.344365) (width 0.2) (layer "F.Cu") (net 14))
 (segment (start 110.38 123.344365) (end 107.88 125.844365) (width 0.2) (layer "F.Cu") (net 14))
 (segment (start 107.88 125.844365) (end 107.88 126.62) (width 0.2) (layer "F.Cu") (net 14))
 (segment (start 107.395 127.105) (end 72.285 127.105) (width 0.2) (layer "F.Cu") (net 14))
 (segment (start 104.5 80.58) (end 110.38 86.46) (width 0.2) (layer "F.Cu") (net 14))
 (segment (start 72.285 127.105) (end 71.18 126) (width 0.2) (layer "F.Cu") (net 14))
 (segment (start 106 99.5) (end 107 100.5) (width 0.2) (layer "F.Cu") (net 12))
 (segment (start 107 100.5) (end 107 103.5) (width 0.2) (layer "F.Cu") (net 12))
 (segment (start 105.5 105) (end 99.8 105) (width 0.2) (layer "F.Cu") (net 12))
 (segment (start 99.8 105) (end 96.58 108.22) (width 0.2) (layer "F.Cu") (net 12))
 (segment (start 107 103.5) (end 105.5 105) (width 0.2) (layer "F.Cu") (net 12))
 (segment (start 104.5 99.5) (end 106 99.5) (width 0.2) (layer "F.Cu") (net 12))
 (segment (start 98.2 99.5) (end 104.5 99.5) (width 0.2) (layer "F.Cu") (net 12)))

